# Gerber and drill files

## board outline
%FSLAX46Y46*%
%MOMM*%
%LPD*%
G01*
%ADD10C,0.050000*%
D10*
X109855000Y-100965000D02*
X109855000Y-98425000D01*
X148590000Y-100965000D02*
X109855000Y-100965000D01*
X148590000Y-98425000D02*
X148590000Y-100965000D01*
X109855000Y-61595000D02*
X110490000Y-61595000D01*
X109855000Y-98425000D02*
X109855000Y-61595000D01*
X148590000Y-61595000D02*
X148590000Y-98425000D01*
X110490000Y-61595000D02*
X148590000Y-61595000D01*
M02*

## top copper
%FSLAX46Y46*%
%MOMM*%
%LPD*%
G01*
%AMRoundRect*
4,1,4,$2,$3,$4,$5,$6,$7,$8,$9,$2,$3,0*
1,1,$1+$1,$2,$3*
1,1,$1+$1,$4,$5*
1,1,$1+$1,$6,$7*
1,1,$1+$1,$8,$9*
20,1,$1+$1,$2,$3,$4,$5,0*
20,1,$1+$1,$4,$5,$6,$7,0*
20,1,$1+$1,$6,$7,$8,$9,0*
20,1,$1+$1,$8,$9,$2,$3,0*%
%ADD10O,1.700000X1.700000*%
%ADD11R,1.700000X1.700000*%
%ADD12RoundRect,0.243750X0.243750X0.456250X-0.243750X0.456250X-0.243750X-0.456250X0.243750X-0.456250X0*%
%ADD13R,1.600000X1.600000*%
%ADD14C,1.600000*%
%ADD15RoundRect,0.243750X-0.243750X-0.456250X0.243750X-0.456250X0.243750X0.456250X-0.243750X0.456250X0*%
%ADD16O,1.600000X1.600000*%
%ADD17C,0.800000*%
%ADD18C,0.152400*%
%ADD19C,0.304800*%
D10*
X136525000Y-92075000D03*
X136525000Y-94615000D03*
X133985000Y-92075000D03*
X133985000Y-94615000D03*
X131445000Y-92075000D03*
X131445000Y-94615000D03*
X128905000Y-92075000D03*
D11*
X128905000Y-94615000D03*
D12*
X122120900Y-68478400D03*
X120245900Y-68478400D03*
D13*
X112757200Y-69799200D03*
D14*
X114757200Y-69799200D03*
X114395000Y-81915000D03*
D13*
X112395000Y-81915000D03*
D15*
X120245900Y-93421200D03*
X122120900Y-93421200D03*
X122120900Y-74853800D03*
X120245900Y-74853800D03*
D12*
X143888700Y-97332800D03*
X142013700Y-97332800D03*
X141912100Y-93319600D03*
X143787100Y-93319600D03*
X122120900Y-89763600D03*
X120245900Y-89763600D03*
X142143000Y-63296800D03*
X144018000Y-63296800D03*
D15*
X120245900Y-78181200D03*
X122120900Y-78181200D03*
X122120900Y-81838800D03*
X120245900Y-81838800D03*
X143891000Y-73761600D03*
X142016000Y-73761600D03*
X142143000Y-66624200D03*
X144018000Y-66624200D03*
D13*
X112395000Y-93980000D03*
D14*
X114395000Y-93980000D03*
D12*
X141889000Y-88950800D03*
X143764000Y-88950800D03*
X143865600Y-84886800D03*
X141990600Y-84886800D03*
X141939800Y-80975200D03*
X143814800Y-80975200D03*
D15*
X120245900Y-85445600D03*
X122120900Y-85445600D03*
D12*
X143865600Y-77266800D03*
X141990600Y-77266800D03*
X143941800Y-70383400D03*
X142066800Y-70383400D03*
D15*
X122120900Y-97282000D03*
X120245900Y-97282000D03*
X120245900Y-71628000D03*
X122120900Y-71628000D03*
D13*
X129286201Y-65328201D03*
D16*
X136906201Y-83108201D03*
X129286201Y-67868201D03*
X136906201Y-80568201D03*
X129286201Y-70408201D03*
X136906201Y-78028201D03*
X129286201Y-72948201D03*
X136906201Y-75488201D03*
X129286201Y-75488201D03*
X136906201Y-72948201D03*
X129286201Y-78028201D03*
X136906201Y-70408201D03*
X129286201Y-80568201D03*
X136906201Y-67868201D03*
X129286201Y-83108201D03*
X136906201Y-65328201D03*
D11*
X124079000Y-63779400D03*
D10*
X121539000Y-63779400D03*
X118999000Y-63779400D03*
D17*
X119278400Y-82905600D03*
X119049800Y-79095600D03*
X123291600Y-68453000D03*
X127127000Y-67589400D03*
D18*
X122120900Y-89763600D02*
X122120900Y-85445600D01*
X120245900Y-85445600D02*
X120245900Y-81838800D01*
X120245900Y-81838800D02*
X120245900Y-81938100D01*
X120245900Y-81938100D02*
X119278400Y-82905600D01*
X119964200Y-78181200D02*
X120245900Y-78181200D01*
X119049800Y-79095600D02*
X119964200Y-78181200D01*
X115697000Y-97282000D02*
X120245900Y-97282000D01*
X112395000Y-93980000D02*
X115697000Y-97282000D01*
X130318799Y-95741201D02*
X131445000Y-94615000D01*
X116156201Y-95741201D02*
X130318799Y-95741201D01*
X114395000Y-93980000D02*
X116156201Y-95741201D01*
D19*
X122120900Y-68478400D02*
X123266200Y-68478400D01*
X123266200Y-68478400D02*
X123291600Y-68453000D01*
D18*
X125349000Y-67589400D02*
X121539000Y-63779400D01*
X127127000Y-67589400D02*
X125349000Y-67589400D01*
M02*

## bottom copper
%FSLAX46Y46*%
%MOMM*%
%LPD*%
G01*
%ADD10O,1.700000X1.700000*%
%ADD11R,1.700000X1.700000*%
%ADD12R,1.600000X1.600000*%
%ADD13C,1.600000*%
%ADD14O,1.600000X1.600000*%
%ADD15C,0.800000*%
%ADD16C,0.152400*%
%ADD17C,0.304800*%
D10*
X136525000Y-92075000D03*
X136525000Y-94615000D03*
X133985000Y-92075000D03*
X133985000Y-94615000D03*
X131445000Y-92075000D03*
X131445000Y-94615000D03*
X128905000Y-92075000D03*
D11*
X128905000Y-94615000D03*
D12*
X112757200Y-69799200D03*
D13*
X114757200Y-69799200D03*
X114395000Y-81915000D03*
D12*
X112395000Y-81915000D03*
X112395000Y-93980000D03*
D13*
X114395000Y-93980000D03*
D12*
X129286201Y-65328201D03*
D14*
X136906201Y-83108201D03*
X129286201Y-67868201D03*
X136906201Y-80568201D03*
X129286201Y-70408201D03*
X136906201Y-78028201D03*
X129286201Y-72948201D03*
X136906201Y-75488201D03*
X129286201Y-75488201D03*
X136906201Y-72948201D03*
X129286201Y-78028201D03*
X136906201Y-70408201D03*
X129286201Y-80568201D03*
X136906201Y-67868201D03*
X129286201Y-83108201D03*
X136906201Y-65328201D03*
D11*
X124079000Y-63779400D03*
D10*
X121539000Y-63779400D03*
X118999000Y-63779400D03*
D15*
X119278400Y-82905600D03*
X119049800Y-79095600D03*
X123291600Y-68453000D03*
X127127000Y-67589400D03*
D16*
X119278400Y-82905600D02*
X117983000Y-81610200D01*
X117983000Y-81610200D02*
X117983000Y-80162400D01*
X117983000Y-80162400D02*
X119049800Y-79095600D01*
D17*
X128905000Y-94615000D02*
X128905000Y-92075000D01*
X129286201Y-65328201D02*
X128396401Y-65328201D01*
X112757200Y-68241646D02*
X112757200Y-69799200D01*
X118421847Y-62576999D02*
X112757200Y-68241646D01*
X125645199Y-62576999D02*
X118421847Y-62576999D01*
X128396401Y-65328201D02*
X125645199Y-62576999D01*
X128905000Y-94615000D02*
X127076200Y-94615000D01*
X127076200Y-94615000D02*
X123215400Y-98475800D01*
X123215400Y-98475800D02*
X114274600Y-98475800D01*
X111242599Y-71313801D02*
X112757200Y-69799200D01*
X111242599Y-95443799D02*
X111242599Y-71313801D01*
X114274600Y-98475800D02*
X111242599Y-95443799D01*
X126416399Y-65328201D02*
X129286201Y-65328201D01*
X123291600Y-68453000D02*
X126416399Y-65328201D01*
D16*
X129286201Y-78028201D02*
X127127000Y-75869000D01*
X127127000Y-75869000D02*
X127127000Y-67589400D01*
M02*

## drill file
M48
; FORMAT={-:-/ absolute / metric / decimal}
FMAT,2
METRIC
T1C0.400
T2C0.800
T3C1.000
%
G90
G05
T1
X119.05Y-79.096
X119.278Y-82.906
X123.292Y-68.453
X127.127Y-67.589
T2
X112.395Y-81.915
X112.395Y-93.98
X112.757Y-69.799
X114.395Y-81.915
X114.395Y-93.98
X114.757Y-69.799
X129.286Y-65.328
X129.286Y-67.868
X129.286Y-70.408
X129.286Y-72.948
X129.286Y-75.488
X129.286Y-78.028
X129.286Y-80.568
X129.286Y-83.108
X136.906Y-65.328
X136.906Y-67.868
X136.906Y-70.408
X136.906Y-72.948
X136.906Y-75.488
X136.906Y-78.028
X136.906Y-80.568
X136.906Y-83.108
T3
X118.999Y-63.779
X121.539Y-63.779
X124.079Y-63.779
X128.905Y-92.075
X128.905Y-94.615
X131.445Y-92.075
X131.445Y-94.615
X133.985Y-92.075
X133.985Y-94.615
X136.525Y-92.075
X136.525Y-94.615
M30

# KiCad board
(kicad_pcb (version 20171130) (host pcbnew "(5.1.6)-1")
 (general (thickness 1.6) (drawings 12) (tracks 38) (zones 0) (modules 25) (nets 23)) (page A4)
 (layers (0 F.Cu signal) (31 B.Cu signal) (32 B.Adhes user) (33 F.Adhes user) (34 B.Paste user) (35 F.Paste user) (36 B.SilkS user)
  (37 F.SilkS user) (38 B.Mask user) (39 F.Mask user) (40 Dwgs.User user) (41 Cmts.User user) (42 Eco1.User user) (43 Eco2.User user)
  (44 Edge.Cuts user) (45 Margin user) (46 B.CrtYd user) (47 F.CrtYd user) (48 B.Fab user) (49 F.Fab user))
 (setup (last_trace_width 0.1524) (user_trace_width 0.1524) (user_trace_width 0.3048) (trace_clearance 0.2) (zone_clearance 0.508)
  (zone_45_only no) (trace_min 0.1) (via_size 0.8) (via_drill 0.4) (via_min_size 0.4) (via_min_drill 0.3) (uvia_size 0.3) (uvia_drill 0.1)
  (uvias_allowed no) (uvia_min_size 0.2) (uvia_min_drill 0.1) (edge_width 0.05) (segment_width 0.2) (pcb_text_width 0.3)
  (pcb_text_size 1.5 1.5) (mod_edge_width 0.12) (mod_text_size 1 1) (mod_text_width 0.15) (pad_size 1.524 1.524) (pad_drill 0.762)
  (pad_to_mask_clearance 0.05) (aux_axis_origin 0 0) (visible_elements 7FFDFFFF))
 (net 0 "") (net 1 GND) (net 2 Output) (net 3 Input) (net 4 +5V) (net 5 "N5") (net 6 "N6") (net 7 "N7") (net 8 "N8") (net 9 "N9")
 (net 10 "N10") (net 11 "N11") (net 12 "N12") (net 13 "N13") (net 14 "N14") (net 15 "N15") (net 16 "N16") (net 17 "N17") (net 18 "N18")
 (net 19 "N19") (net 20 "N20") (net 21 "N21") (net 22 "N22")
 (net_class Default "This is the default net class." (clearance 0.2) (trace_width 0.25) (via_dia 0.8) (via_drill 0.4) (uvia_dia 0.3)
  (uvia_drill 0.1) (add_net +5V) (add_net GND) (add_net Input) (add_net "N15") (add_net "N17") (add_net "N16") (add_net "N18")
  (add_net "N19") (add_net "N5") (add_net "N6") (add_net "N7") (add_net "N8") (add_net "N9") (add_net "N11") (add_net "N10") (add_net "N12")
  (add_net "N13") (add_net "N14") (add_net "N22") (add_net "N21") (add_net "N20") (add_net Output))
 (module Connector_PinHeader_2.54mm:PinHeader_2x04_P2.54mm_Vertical (layer F.Cu) (at 128.905 94.615 90)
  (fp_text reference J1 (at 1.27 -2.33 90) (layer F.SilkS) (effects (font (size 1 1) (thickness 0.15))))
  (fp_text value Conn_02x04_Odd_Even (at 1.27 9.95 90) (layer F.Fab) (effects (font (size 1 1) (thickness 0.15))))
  (pad 8 thru_hole oval (at 2.54 7.62 90) (size 1.7 1.7) (drill 1) (layers *.Cu *.Mask) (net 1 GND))
  (pad 7 thru_hole oval (at 0 7.62 90) (size 1.7 1.7) (drill 1) (layers *.Cu *.Mask) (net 1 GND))
  (pad 6 thru_hole oval (at 2.54 5.08 90) (size 1.7 1.7) (drill 1) (layers *.Cu *.Mask) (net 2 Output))
  (pad 5 thru_hole oval (at 0 5.08 90) (size 1.7 1.7) (drill 1) (layers *.Cu *.Mask) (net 2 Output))
  (pad 4 thru_hole oval (at 2.54 2.54 90) (size 1.7 1.7) (drill 1) (layers *.Cu *.Mask) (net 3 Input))
  (pad 3 thru_hole oval (at 0 2.54 90) (size 1.7 1.7) (drill 1) (layers *.Cu *.Mask) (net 3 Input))
  (pad 2 thru_hole oval (at 2.54 0 90) (size 1.7 1.7) (drill 1) (layers *.Cu *.Mask) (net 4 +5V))
  (pad 1 thru_hole rect (at 0 0 90) (size 1.7 1.7) (drill 1) (layers *.Cu *.Mask) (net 4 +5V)))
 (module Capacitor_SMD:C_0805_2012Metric (layer F.Cu) (at 121.1834 68.4784 180)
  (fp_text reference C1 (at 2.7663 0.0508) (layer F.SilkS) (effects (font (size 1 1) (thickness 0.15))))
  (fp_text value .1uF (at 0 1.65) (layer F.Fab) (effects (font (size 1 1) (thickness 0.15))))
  (pad 1 smd roundrect (at -0.9375 0 180) (size 0.975 1.4) (layers F.Cu F.Paste F.Mask) (roundrect_rratio 0.25) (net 4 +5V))
  (pad 2 smd roundrect (at 0.9375 0 180) (size 0.975 1.4) (layers F.Cu F.Paste F.Mask) (roundrect_rratio 0.25) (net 1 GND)))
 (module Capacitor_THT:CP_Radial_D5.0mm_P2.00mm (layer F.Cu) (at 112.7572 69.7992)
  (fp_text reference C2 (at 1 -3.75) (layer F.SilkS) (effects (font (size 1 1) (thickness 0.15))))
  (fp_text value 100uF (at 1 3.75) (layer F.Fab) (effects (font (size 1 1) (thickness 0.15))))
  (pad 1 thru_hole rect (at 0 0) (size 1.6 1.6) (drill 0.8) (layers *.Cu *.Mask) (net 4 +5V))
  (pad 2 thru_hole circle (at 2 0) (size 1.6 1.6) (drill 0.8) (layers *.Cu *.Mask) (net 1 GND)))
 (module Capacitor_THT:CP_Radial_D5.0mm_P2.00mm (layer F.Cu) (at 112.395 81.915)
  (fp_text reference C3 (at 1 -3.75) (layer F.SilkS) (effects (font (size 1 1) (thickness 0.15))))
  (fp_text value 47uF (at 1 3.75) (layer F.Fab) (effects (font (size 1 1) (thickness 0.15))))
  (pad 2 thru_hole circle (at 2 0) (size 1.6 1.6) (drill 0.8) (layers *.Cu *.Mask) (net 1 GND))
  (pad 1 thru_hole rect (at 0 0) (size 1.6 1.6) (drill 0.8) (layers *.Cu *.Mask) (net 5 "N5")))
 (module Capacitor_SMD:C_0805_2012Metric (layer F.Cu) (at 121.1834 93.4212)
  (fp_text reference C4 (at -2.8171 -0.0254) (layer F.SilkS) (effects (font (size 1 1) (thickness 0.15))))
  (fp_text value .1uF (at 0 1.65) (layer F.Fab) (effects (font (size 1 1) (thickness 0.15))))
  (pad 1 smd roundrect (at -0.9375 0) (size 0.975 1.4) (layers F.Cu F.Paste F.Mask) (roundrect_rratio 0.25) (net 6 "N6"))
  (pad 2 smd roundrect (at 0.9375 0) (size 0.975 1.4) (layers F.Cu F.Paste F.Mask) (roundrect_rratio 0.25) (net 1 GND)))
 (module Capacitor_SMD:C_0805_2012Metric (layer F.Cu) (at 121.1834 74.8538)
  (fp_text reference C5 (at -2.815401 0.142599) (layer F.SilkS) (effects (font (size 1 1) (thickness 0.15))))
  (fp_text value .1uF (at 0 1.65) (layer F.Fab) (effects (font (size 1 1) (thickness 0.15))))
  (pad 2 smd roundrect (at 0.9375 0) (size 0.975 1.4) (layers F.Cu F.Paste F.Mask) (roundrect_rratio 0.25) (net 1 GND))
  (pad 1 smd roundrect (at -0.9375 0) (size 0.975 1.4) (layers F.Cu F.Paste F.Mask) (roundrect_rratio 0.25) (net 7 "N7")))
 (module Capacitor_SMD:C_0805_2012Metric (layer F.Cu) (at 142.9512 97.3328 180)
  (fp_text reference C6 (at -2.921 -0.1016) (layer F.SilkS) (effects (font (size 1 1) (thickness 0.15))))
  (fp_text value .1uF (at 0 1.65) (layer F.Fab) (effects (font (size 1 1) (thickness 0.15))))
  (pad 1 smd roundrect (at -0.9375 0 180) (size 0.975 1.4) (layers F.Cu F.Paste F.Mask) (roundrect_rratio 0.25) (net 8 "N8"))
  (pad 2 smd roundrect (at 0.9375 0 180) (size 0.975 1.4) (layers F.Cu F.Paste F.Mask) (roundrect_rratio 0.25) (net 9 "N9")))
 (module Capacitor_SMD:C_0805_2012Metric (layer F.Cu) (at 142.8496 93.3196 180)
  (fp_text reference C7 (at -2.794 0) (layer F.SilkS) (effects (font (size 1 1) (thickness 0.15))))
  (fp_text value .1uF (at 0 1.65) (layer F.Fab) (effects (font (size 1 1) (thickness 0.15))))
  (pad 2 smd roundrect (at 0.9375 0 180) (size 0.975 1.4) (layers F.Cu F.Paste F.Mask) (roundrect_rratio 0.25) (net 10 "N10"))
  (pad 1 smd roundrect (at -0.9375 0 180) (size 0.975 1.4) (layers F.Cu F.Paste F.Mask) (roundrect_rratio 0.25) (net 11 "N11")))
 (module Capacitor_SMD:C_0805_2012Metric (layer F.Cu) (at 121.1834 89.7636 180)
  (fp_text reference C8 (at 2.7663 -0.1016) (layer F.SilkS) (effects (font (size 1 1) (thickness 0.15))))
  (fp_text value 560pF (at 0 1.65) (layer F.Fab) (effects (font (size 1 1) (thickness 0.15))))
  (pad 1 smd roundrect (at -0.9375 0 180) (size 0.975 1.4) (layers F.Cu F.Paste F.Mask) (roundrect_rratio 0.25) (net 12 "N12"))
  (pad 2 smd roundrect (at 0.9375 0 180) (size 0.975 1.4) (layers F.Cu F.Paste F.Mask) (roundrect_rratio 0.25) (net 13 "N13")))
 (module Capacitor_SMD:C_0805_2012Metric (layer F.Cu) (at 143.0805 63.2968 180)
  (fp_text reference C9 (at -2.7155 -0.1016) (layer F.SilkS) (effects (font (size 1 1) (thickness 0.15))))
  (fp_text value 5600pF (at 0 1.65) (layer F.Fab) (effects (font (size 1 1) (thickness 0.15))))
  (pad 2 smd roundrect (at 0.9375 0 180) (size 0.975 1.4) (layers F.Cu F.Paste F.Mask) (roundrect_rratio 0.25) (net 1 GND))
  (pad 1 smd roundrect (at -0.9375 0 180) (size 0.975 1.4) (layers F.Cu F.Paste F.Mask) (roundrect_rratio 0.25) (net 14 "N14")))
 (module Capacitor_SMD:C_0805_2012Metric (layer F.Cu) (at 121.1834 78.1812)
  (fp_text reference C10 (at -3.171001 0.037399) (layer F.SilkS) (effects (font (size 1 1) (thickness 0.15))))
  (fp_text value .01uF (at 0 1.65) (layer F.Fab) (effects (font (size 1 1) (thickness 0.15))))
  (pad 1 smd roundrect (at -0.9375 0) (size 0.975 1.4) (layers F.Cu F.Paste F.Mask) (roundrect_rratio 0.25) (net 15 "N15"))
  (pad 2 smd roundrect (at 0.9375 0) (size 0.975 1.4) (layers F.Cu F.Paste F.Mask) (roundrect_rratio 0.25) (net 1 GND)))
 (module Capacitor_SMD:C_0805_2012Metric (layer F.Cu) (at 121.1834 81.8388)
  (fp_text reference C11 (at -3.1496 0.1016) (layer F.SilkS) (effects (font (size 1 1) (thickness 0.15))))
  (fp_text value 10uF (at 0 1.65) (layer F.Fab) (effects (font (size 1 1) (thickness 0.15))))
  (pad 2 smd roundrect (at 0.9375 0) (size 0.975 1.4) (layers F.Cu F.Paste F.Mask) (roundrect_rratio 0.25) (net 2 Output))
  (pad 1 smd roundrect (at -0.9375 0) (size 0.975 1.4) (layers F.Cu F.Paste F.Mask) (roundrect_rratio 0.25) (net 15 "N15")))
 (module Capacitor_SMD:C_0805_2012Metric (layer F.Cu) (at 142.9535 73.7616)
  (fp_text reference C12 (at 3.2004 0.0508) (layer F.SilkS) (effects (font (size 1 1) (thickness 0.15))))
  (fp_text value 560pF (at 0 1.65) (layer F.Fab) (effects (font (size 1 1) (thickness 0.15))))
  (pad 2 smd roundrect (at 0.9375 0) (size 0.975 1.4) (layers F.Cu F.Paste F.Mask) (roundrect_rratio 0.25) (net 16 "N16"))
  (pad 1 smd roundrect (at -0.9375 0) (size 0.975 1.4) (layers F.Cu F.Paste F.Mask) (roundrect_rratio 0.25) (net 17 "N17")))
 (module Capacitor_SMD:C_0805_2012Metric (layer F.Cu) (at 143.0805 66.6242)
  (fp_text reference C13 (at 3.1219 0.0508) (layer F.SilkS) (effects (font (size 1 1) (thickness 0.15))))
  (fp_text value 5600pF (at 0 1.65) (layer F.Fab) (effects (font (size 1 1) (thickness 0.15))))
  (pad 1 smd roundrect (at -0.9375 0) (size 0.975 1.4) (layers F.Cu F.Paste F.Mask) (roundrect_rratio 0.25) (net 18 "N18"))
  (pad 2 smd roundrect (at 0.9375 0) (size 0.975 1.4) (layers F.Cu F.Paste F.Mask) (roundrect_rratio 0.25) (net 1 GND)))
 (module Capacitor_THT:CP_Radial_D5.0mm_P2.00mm (layer F.Cu) (at 112.395 93.98)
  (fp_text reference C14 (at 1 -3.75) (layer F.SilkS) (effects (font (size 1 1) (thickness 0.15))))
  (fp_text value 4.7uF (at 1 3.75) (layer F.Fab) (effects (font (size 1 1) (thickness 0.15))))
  (pad 1 thru_hole rect (at 0 0) (size 1.6 1.6) (drill 0.8) (layers *.Cu *.Mask) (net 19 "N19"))
  (pad 2 thru_hole circle (at 2 0) (size 1.6 1.6) (drill 0.8) (layers *.Cu *.Mask) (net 3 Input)))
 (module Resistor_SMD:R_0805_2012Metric (layer F.Cu) (at 142.8265 88.9508 180)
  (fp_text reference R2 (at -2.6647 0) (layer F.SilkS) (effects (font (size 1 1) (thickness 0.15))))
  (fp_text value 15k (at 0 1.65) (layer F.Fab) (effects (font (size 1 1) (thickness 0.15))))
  (pad 2 smd roundrect (at 0.9375 0 180) (size 0.975 1.4) (layers F.Cu F.Paste F.Mask) (roundrect_rratio 0.25) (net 11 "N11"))
  (pad 1 smd roundrect (at -0.9375 0 180) (size 0.975 1.4) (layers F.Cu F.Paste F.Mask) (roundrect_rratio 0.25) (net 14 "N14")))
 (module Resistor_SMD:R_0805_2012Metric (layer F.Cu) (at 142.9281 84.8868 180)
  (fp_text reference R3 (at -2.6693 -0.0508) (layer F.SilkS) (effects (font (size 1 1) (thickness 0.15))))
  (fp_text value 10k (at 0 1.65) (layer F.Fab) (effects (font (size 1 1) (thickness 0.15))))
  (pad 1 smd roundrect (at -0.9375 0 180) (size 0.975 1.4) (layers F.Cu F.Paste F.Mask) (roundrect_rratio 0.25) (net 14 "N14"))
  (pad 2 smd roundrect (at 0.9375 0 180) (size 0.975 1.4) (layers F.Cu F.Paste F.Mask) (roundrect_rratio 0.25) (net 13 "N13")))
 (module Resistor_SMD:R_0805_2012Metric (layer F.Cu) (at 142.8773 80.9752 180)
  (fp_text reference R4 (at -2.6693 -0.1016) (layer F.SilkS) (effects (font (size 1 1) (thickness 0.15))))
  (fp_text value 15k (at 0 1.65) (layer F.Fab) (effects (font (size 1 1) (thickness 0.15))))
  (pad 2 smd roundrect (at 0.9375 0 180) (size 0.975 1.4) (layers F.Cu F.Paste F.Mask) (roundrect_rratio 0.25) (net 12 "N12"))
  (pad 1 smd roundrect (at -0.9375 0 180) (size 0.975 1.4) (layers F.Cu F.Paste F.Mask) (roundrect_rratio 0.25) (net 14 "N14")))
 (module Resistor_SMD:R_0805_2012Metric (layer F.Cu) (at 121.1834 85.4456)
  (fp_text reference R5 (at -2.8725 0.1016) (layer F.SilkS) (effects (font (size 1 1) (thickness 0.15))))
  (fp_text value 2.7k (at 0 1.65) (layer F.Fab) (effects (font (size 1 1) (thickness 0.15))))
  (pad 1 smd roundrect (at -0.9375 0) (size 0.975 1.4) (layers F.Cu F.Paste F.Mask) (roundrect_rratio 0.25) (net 15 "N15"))
  (pad 2 smd roundrect (at 0.9375 0) (size 0.975 1.4) (layers F.Cu F.Paste F.Mask) (roundrect_rratio 0.25) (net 12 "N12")))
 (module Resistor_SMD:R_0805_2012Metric (layer F.Cu) (at 142.9281 77.2668 180)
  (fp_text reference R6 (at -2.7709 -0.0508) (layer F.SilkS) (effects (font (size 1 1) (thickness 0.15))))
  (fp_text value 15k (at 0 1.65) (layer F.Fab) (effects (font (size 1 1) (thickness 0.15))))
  (pad 1 smd roundrect (at -0.9375 0 180) (size 0.975 1.4) (layers F.Cu F.Paste F.Mask) (roundrect_rratio 0.25) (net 18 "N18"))
  (pad 2 smd roundrect (at 0.9375 0 180) (size 0.975 1.4) (layers F.Cu F.Paste F.Mask) (roundrect_rratio 0.25) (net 16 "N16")))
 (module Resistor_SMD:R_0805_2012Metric (layer F.Cu) (at 143.0043 70.3834 180)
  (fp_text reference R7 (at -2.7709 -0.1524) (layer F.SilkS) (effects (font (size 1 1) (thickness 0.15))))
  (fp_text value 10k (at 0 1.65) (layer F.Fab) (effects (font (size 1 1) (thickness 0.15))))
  (pad 1 smd roundrect (at -0.9375 0 180) (size 0.975 1.4) (layers F.Cu F.Paste F.Mask) (roundrect_rratio 0.25) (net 18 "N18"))
  (pad 2 smd roundrect (at 0.9375 0 180) (size 0.975 1.4) (layers F.Cu F.Paste F.Mask) (roundrect_rratio 0.25) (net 17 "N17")))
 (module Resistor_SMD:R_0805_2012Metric (layer F.Cu) (at 121.1834 97.282)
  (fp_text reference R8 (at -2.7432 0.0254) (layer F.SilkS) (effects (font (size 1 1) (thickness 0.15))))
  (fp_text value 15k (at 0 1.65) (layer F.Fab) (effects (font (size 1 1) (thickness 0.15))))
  (pad 2 smd roundrect (at 0.9375 0) (size 0.975 1.4) (layers F.Cu F.Paste F.Mask) (roundrect_rratio 0.25) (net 18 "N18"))
  (pad 1 smd roundrect (at -0.9375 0) (size 0.975 1.4) (layers F.Cu F.Paste F.Mask) (roundrect_rratio 0.25) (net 19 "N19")))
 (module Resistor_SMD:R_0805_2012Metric (layer F.Cu) (at 121.1834 71.628)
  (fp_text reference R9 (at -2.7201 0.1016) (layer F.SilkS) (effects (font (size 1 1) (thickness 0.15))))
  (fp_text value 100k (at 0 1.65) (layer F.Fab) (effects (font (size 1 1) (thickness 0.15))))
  (pad 1 smd roundrect (at -0.9375 0) (size 0.975 1.4) (layers F.Cu F.Paste F.Mask) (roundrect_rratio 0.25) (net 1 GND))
  (pad 2 smd roundrect (at 0.9375 0) (size 0.975 1.4) (layers F.Cu F.Paste F.Mask) (roundrect_rratio 0.25) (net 3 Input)))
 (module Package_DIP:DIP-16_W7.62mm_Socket (layer F.Cu) (at 129.286201 65.328201)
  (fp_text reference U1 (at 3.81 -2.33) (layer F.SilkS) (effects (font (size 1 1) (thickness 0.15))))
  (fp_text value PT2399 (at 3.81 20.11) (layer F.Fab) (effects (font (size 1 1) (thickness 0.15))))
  (pad 1 thru_hole rect (at 0 0) (size 1.6 1.6) (drill 0.8) (layers *.Cu *.Mask) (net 4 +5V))
  (pad 9 thru_hole oval (at 7.62 17.78) (size 1.6 1.6) (drill 0.8) (layers *.Cu *.Mask) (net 9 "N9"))
  (pad 2 thru_hole oval (at 0 2.54) (size 1.6 1.6) (drill 0.8) (layers *.Cu *.Mask) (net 5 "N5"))
  (pad 10 thru_hole oval (at 7.62 15.24) (size 1.6 1.6) (drill 0.8) (layers *.Cu *.Mask) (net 8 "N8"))
  (pad 3 thru_hole oval (at 0 5.08) (size 1.6 1.6) (drill 0.8) (layers *.Cu *.Mask) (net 1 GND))
  (pad 11 thru_hole oval (at 7.62 12.7) (size 1.6 1.6) (drill 0.8) (layers *.Cu *.Mask) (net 10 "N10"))
  (pad 4 thru_hole oval (at 0 7.62) (size 1.6 1.6) (drill 0.8) (layers *.Cu *.Mask) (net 1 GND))
  (pad 12 thru_hole oval (at 7.62 10.16) (size 1.6 1.6) (drill 0.8) (layers *.Cu *.Mask) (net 10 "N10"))
  (pad 5 thru_hole oval (at 0 10.16) (size 1.6 1.6) (drill 0.8) (layers *.Cu *.Mask) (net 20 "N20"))
  (pad 13 thru_hole oval (at 7.62 7.62) (size 1.6 1.6) (drill 0.8) (layers *.Cu *.Mask) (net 13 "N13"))
  (pad 6 thru_hole oval (at 0 12.7) (size 1.6 1.6) (drill 0.8) (layers *.Cu *.Mask) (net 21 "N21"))
  (pad 14 thru_hole oval (at 7.62 5.08) (size 1.6 1.6) (drill 0.8) (layers *.Cu *.Mask) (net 12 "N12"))
  (pad 7 thru_hole oval (at 0 15.24) (size 1.6 1.6) (drill 0.8) (layers *.Cu *.Mask) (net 6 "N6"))
  (pad 15 thru_hole oval (at 7.62 2.54) (size 1.6 1.6) (drill 0.8) (layers *.Cu *.Mask) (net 16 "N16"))
  (pad 8 thru_hole oval (at 0 17.78) (size 1.6 1.6) (drill 0.8) (layers *.Cu *.Mask) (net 7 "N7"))
  (pad 16 thru_hole oval (at 7.62 0) (size 1.6 1.6) (drill 0.8) (layers *.Cu *.Mask) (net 17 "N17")))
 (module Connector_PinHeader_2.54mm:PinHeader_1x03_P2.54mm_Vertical (layer F.Cu) (at 124.079 63.7794 270)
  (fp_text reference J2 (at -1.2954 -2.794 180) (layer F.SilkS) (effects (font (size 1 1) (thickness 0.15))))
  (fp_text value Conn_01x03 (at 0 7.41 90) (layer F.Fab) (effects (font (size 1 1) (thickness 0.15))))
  (pad 1 thru_hole rect (at 0 0 270) (size 1.7 1.7) (drill 1) (layers *.Cu *.Mask) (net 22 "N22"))
  (pad 2 thru_hole oval (at 0 2.54 270) (size 1.7 1.7) (drill 1) (layers *.Cu *.Mask) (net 21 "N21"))
  (pad 3 thru_hole oval (at 0 5.08 270) (size 1.7 1.7) (drill 1) (layers *.Cu *.Mask) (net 1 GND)))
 (gr_line (start 109.855 100.965) (end 109.855 98.425) (layer Edge.Cuts) (width 0.05))
 (gr_line (start 148.59 100.965) (end 109.855 100.965) (layer Edge.Cuts) (width 0.05))
 (gr_line (start 148.59 98.425) (end 148.59 100.965) (layer Edge.Cuts) (width 0.05))
 (gr_line (start 109.855 61.595) (end 110.49 61.595) (layer Edge.Cuts) (width 0.05))
 (gr_line (start 109.855 98.425) (end 109.855 61.595) (layer Edge.Cuts) (width 0.05))
 (gr_line (start 148.59 61.595) (end 148.59 98.425) (layer Edge.Cuts) (width 0.05))
 (gr_line (start 110.49 61.595) (end 148.59 61.595) (layer Edge.Cuts) (width 0.05))
 (segment (start 122.1209 89.7636) (end 122.1209 85.4456) (width 0.1524) (layer F.Cu) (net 12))
 (segment (start 120.2459 85.4456) (end 120.2459 81.8388) (width 0.1524) (layer F.Cu) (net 15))
 (via (at 119.2784 82.9056) (size 0.8) (drill 0.4) (layers F.Cu B.Cu) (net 15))
 (segment (start 120.2459 81.8388) (end 120.2459 81.9381) (width 0.1524) (layer F.Cu) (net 15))
 (segment (start 120.2459 81.9381) (end 119.2784 82.9056) (width 0.1524) (layer F.Cu) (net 15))
 (segment (start 119.2784 82.9056) (end 117.983 81.6102) (width 0.1524) (layer B.Cu) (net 15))
 (via (at 119.0498 79.0956) (size 0.8) (drill 0.4) (layers F.Cu B.Cu) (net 15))
 (segment (start 117.983 81.6102) (end 117.983 80.1624) (width 0.1524) (layer B.Cu) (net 15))
 (segment (start 117.983 80.1624) (end 119.0498 79.0956) (width 0.1524) (layer B.Cu) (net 15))
 (segment (start 119.9642 78.1812) (end 120.2459 78.1812) (width 0.1524) (layer F.Cu) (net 15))
 (segment (start 119.0498 79.0956) (end 119.9642 78.1812) (width 0.1524) (layer F.Cu) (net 15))
 (segment (start 115.697 97.282) (end 120.2459 97.282) (width 0.1524) (layer F.Cu) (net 19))
 (segment (start 112.395 93.98) (end 115.697 97.282) (width 0.1524) (layer F.Cu) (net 19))
 (segment (start 130.318799 95.741201) (end 131.445 94.615) (width 0.1524) (layer F.Cu) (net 3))
 (segment (start 116.156201 95.741201) (end 130.318799 95.741201) (width 0.1524) (layer F.Cu) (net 3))
 (segment (start 114.395 93.98) (end 116.156201 95.741201) (width 0.1524) (layer F.Cu) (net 3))
 (segment (start 128.905 94.615) (end 128.905 92.075) (width 0.3048) (layer B.Cu) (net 4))
 (segment (start 129.286201 65.328201) (end 128.396401 65.328201) (width 0.3048) (layer B.Cu) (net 4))
 (segment (start 112.7572 68.241646) (end 112.7572 69.7992) (width 0.3048) (layer B.Cu) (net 4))
 (segment (start 118.421847 62.576999) (end 112.7572 68.241646) (width 0.3048) (layer B.Cu) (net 4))
 (segment (start 125.645199 62.576999) (end 118.421847 62.576999) (width 0.3048) (layer B.Cu) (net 4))
 (segment (start 128.396401 65.328201) (end 125.645199 62.576999) (width 0.3048) (layer B.Cu) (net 4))
 (segment (start 128.905 94.615) (end 127.0762 94.615) (width 0.3048) (layer B.Cu) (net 4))
 (segment (start 127.0762 94.615) (end 123.2154 98.4758) (width 0.3048) (layer B.Cu) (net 4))
 (segment (start 123.2154 98.4758) (end 114.2746 98.4758) (width 0.3048) (layer B.Cu) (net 4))
 (segment (start 111.242599 71.313801) (end 112.7572 69.7992) (width 0.3048) (layer B.Cu) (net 4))
 (segment (start 111.242599 95.443799) (end 111.242599 71.313801) (width 0.3048) (layer B.Cu) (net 4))
 (segment (start 114.2746 98.4758) (end 111.242599 95.443799) (width 0.3048) (layer B.Cu) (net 4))
 (via (at 123.2916 68.453) (size 0.8) (drill 0.4) (layers F.Cu B.Cu) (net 4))
 (segment (start 122.1209 68.4784) (end 123.2662 68.4784) (width 0.3048) (layer F.Cu) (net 4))
 (segment (start 123.2662 68.4784) (end 123.2916 68.453) (width 0.3048) (layer F.Cu) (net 4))
 (segment (start 126.416399 65.328201) (end 129.286201 65.328201) (width 0.3048) (layer B.Cu) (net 4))
 (segment (start 123.2916 68.453) (end 126.416399 65.328201) (width 0.3048) (layer B.Cu) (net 4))
 (via (at 127.127 67.5894) (size 0.8) (drill 0.4) (layers F.Cu B.Cu) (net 21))
 (segment (start 129.286201 78.028201) (end 127.127 75.869) (width 0.1524) (layer B.Cu) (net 21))
 (segment (start 127.127 75.869) (end 127.127 67.5894) (width 0.1524) (layer B.Cu) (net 21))
 (segment (start 125.349 67.5894) (end 121.539 63.7794) (width 0.1524) (layer F.Cu) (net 21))
 (segment (start 127.127 67.5894) (end 125.349 67.5894) (width 0.1524) (layer F.Cu) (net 21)))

